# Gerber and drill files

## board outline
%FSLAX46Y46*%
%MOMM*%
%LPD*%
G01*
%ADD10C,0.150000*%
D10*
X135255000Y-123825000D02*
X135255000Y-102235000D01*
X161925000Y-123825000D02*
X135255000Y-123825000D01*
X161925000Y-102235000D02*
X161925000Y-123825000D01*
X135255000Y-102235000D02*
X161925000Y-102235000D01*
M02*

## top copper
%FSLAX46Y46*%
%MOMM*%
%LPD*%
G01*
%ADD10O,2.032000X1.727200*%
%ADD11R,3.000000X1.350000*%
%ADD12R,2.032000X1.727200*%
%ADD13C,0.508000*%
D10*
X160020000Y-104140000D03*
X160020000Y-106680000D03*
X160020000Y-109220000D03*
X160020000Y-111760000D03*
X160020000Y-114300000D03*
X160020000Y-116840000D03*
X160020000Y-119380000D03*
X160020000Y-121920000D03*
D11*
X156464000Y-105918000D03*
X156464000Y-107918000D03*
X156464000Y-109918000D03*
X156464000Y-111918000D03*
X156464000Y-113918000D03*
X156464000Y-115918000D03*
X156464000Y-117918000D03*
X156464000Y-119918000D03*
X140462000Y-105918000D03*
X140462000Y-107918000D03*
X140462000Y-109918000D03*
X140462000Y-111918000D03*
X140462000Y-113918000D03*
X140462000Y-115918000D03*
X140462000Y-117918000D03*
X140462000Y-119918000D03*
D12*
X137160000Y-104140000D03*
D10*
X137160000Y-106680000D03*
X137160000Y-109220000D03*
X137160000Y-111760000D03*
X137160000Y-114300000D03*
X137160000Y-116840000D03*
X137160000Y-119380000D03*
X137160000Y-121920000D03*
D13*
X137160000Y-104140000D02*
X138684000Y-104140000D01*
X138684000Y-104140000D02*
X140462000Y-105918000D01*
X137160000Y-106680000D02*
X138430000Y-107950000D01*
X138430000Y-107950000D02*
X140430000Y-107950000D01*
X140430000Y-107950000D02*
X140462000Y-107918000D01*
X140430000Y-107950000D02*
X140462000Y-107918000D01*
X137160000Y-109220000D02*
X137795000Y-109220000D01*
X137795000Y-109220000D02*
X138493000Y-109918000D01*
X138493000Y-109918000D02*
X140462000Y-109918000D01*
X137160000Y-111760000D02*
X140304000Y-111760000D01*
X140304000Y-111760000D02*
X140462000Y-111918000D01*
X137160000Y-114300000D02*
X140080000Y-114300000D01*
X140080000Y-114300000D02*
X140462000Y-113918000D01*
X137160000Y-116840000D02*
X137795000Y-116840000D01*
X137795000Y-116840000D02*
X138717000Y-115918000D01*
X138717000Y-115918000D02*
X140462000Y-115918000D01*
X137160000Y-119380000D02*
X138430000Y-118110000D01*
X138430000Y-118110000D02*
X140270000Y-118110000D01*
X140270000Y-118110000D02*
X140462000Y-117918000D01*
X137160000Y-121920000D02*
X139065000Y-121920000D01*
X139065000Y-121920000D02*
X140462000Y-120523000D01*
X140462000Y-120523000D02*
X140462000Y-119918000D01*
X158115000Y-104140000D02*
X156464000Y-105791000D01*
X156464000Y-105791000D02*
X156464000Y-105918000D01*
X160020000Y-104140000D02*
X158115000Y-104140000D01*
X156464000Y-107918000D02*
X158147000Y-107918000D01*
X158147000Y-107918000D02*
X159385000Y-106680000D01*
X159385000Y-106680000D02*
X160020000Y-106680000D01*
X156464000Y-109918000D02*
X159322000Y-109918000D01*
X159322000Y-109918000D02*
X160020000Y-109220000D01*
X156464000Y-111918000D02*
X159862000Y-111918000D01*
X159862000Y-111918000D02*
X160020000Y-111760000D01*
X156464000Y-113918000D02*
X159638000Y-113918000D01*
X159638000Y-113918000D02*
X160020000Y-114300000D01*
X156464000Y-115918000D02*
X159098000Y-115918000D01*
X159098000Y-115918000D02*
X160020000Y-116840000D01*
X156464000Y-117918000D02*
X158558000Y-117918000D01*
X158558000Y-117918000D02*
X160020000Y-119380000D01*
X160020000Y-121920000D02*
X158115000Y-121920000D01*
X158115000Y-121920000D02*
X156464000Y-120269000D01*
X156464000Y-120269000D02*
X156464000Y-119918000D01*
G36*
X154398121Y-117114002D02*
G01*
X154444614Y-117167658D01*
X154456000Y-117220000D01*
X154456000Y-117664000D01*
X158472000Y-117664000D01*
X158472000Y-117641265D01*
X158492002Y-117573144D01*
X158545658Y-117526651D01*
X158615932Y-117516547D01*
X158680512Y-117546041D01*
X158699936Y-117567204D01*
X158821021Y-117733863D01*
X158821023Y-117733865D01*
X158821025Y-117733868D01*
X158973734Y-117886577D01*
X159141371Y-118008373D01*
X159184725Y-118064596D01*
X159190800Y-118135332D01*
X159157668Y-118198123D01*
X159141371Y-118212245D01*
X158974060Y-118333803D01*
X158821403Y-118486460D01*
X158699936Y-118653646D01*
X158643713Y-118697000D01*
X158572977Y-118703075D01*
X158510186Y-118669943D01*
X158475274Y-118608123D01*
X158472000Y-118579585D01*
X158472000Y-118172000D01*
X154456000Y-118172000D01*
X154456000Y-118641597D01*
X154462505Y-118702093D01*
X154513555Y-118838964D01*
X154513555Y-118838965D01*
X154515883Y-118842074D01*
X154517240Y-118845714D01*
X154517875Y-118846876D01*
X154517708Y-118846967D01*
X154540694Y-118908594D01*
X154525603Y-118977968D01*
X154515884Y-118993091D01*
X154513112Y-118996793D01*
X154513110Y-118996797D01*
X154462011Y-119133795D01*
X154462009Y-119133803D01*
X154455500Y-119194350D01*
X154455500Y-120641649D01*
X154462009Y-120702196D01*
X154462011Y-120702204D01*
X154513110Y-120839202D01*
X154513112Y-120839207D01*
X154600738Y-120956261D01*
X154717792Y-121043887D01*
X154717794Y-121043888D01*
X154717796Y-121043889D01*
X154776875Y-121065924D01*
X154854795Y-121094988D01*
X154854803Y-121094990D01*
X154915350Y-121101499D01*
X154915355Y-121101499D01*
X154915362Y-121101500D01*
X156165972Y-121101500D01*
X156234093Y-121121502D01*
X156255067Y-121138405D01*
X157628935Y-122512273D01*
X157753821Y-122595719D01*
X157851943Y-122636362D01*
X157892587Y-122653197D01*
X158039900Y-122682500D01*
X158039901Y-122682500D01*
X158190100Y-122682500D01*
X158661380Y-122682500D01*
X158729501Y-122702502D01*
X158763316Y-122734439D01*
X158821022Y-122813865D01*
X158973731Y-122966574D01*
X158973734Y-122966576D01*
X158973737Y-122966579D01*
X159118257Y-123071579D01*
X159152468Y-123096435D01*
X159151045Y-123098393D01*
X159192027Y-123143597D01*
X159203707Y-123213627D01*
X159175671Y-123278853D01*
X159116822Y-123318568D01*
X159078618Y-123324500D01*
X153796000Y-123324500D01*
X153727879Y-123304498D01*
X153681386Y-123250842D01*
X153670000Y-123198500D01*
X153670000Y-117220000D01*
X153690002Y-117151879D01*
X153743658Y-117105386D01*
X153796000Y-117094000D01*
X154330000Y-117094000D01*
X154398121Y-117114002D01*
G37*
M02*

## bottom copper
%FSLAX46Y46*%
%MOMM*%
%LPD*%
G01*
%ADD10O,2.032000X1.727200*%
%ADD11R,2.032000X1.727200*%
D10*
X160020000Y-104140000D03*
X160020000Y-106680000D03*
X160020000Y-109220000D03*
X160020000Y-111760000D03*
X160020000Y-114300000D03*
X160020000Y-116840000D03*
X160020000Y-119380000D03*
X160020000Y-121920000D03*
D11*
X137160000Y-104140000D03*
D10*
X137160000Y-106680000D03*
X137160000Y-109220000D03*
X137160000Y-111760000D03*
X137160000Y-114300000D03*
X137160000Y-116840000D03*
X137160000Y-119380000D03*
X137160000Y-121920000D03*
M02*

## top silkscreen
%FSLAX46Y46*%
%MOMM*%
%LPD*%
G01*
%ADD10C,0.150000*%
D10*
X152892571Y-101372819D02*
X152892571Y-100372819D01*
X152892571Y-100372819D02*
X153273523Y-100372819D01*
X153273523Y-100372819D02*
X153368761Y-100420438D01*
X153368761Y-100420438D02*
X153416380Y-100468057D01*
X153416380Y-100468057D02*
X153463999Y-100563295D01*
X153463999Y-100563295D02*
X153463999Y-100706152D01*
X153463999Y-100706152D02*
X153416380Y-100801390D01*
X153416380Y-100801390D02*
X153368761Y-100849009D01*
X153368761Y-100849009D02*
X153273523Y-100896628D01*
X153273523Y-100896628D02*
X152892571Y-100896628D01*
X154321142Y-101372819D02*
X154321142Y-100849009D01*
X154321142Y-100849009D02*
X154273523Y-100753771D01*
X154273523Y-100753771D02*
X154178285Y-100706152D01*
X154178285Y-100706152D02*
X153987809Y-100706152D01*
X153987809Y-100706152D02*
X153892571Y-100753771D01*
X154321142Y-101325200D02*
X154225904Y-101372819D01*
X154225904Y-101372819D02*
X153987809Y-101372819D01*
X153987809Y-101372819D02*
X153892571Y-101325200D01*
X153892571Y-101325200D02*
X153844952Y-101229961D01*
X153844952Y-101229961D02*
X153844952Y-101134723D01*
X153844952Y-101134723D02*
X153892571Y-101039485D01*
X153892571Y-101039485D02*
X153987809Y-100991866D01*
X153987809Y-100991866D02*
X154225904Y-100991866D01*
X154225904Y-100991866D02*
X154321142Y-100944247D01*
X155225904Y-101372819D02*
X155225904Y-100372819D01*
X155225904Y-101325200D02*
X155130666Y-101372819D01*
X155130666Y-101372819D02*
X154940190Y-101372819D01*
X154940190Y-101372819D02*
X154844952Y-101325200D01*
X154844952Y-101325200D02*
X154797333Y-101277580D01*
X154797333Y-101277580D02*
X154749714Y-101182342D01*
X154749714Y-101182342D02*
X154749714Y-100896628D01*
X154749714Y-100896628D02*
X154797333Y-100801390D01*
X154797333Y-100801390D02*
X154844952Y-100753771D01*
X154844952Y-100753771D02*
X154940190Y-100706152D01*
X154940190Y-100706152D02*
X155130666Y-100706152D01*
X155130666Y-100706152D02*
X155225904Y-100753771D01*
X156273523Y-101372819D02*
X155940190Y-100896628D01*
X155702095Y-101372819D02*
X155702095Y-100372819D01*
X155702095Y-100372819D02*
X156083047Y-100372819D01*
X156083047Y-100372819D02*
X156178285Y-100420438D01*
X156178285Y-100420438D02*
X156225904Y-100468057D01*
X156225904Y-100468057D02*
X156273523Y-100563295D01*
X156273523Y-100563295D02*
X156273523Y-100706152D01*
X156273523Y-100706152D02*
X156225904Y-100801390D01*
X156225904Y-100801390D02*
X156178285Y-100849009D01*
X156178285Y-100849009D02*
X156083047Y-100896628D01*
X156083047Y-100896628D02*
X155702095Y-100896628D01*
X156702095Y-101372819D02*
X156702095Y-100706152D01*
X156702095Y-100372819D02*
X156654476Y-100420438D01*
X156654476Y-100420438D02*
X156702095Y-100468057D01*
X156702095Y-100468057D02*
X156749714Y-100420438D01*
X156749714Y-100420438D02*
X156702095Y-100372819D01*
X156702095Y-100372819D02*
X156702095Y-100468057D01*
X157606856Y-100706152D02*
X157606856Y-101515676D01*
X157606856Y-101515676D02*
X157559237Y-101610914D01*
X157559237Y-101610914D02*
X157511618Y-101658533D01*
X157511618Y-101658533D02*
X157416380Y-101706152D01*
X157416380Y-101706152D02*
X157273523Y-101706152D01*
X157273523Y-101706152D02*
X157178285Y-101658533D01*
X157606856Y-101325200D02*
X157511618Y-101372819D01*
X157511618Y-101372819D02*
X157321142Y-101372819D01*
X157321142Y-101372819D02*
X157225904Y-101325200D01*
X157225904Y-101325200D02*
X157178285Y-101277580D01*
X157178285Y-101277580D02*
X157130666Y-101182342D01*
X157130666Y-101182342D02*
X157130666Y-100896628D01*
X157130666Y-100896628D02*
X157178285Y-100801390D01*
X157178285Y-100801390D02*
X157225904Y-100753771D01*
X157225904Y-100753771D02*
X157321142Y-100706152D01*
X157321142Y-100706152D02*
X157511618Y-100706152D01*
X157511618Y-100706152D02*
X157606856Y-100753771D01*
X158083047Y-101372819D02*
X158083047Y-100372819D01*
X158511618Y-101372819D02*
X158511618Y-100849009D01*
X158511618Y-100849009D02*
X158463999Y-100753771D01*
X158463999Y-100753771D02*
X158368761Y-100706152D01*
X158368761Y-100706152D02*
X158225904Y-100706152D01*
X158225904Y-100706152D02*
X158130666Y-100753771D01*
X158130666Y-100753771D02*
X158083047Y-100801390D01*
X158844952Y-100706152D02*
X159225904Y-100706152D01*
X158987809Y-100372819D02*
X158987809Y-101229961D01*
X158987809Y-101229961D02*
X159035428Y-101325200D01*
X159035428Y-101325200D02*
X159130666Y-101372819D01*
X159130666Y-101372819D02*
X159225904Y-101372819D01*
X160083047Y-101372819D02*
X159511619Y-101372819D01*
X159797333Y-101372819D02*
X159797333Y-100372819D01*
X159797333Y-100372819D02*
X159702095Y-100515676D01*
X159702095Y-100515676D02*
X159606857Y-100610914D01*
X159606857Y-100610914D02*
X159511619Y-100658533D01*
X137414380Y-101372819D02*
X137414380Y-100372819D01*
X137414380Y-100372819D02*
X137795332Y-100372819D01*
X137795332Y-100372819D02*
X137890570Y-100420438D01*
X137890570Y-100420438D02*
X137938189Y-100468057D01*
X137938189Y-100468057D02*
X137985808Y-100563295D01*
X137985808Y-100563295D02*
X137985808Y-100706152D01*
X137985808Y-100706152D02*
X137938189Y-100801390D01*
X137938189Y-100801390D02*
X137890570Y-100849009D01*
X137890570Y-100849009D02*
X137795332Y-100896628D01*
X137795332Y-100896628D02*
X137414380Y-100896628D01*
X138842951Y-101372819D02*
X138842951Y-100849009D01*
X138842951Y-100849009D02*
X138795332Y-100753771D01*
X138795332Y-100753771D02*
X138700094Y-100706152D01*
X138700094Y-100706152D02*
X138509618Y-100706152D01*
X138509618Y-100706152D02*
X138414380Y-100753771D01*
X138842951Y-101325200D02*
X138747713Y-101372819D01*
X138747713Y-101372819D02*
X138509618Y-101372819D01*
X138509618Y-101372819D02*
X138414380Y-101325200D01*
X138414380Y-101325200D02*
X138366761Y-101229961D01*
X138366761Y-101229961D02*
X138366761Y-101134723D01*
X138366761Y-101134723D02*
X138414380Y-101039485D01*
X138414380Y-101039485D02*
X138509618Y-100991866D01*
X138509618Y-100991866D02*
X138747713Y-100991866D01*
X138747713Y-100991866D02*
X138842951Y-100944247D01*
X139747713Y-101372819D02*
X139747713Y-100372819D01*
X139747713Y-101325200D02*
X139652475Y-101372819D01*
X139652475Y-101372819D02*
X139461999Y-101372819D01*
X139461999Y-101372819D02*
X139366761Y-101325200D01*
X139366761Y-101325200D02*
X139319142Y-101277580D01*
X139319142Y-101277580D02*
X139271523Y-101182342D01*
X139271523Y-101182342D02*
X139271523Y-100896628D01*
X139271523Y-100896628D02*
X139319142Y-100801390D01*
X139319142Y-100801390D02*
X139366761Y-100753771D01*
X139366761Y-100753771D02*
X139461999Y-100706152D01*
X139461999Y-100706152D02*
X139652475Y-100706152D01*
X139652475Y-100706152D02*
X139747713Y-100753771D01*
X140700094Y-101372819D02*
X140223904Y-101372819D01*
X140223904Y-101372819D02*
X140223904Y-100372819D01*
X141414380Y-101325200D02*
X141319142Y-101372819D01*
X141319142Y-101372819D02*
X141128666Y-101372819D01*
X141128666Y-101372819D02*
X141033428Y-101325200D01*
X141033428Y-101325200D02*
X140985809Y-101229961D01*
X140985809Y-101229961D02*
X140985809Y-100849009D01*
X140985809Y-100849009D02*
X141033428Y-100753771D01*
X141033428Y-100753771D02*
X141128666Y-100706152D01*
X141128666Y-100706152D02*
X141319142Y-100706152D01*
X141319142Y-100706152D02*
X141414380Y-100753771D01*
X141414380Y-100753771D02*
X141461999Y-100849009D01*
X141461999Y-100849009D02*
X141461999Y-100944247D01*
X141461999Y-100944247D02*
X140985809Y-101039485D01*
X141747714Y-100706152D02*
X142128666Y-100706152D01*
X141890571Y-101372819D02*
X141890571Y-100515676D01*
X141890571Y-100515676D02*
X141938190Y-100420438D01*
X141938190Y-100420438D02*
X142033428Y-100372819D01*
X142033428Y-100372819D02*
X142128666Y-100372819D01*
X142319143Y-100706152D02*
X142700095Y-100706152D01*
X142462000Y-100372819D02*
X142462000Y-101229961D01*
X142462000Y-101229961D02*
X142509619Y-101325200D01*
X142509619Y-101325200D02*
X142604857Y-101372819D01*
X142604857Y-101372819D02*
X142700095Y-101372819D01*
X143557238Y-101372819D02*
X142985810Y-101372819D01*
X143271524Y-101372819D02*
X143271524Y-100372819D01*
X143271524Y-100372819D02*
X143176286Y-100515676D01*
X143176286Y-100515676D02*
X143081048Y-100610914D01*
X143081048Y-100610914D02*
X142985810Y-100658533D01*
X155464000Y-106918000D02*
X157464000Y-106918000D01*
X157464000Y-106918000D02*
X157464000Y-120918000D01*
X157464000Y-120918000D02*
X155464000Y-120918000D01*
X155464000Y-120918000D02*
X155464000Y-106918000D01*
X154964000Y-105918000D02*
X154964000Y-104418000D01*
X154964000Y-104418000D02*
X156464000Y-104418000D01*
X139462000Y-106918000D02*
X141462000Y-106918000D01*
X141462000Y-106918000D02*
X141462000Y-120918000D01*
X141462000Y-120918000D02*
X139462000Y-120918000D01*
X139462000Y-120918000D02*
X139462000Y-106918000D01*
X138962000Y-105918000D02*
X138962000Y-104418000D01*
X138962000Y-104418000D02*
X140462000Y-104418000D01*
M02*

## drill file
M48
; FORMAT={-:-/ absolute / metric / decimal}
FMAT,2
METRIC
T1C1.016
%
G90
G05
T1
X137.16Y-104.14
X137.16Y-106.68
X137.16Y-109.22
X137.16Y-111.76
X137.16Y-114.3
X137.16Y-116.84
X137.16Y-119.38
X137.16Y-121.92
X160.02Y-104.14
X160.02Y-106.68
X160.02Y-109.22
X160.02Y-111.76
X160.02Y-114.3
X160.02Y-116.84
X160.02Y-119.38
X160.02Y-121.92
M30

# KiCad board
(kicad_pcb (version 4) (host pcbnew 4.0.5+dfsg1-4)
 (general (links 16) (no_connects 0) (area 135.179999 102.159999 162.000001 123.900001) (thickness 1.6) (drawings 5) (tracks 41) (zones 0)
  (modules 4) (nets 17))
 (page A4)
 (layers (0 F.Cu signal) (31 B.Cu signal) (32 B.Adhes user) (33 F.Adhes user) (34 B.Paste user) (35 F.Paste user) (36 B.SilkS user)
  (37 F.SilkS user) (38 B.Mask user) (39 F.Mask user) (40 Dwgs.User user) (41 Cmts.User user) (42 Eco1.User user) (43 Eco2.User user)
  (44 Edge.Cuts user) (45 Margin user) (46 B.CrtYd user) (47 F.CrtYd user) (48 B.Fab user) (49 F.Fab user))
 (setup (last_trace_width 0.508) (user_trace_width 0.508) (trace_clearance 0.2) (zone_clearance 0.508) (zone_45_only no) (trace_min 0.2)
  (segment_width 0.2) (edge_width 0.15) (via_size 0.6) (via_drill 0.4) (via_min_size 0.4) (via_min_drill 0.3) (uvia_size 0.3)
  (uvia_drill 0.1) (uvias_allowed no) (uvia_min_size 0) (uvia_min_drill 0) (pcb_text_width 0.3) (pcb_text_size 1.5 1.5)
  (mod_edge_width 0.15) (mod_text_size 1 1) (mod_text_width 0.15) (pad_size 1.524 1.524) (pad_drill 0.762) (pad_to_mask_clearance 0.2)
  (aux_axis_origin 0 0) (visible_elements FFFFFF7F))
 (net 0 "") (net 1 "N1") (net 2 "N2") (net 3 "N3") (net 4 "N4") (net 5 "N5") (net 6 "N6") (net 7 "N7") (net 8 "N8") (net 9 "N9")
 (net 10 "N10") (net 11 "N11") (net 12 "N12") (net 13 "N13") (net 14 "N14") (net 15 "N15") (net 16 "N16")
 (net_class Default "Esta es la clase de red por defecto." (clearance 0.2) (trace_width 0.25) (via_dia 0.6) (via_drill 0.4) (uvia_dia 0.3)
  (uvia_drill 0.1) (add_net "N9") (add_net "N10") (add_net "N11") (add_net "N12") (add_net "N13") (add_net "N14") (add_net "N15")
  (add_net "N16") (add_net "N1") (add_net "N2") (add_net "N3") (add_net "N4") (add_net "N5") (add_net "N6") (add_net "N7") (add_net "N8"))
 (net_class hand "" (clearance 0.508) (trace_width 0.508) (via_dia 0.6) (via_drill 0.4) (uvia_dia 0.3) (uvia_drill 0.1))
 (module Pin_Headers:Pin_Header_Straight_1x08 (layer B.Cu) (at 160.02 104.14 180)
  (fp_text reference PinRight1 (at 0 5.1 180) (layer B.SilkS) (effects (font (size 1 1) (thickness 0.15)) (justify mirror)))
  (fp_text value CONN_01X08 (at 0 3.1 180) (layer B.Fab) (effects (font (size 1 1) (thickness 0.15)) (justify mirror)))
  (pad 1 thru_hole oval (at 0 0 180) (size 2.032 1.7272) (drill 1.016) (layers *.Cu *.Mask) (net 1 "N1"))
  (pad 2 thru_hole oval (at 0 -2.54 180) (size 2.032 1.7272) (drill 1.016) (layers *.Cu *.Mask) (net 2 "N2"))
  (pad 3 thru_hole oval (at 0 -5.08 180) (size 2.032 1.7272) (drill 1.016) (layers *.Cu *.Mask) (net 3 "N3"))
  (pad 4 thru_hole oval (at 0 -7.62 180) (size 2.032 1.7272) (drill 1.016) (layers *.Cu *.Mask) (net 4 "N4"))
  (pad 5 thru_hole oval (at 0 -10.16 180) (size 2.032 1.7272) (drill 1.016) (layers *.Cu *.Mask) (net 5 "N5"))
  (pad 6 thru_hole oval (at 0 -12.7 180) (size 2.032 1.7272) (drill 1.016) (layers *.Cu *.Mask) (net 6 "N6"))
  (pad 7 thru_hole oval (at 0 -15.24 180) (size 2.032 1.7272) (drill 1.016) (layers *.Cu *.Mask) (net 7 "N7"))
  (pad 8 thru_hole oval (at 0 -17.78 180) (size 2.032 1.7272) (drill 1.016) (layers *.Cu *.Mask) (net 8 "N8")))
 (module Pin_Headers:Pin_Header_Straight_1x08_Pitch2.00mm (layer F.Cu) (at 156.464 105.918)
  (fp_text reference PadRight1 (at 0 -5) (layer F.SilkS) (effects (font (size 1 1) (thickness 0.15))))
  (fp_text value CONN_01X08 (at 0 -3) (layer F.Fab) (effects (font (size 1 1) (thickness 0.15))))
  (fp_line (start -1 1) (end 1 1) (layer F.SilkS) (width 0.15))
  (fp_line (start 1 1) (end 1 15) (layer F.SilkS) (width 0.15))
  (fp_line (start 1 15) (end -1 15) (layer F.SilkS) (width 0.15))
  (fp_line (start -1 15) (end -1 1) (layer F.SilkS) (width 0.15))
  (fp_line (start -1.5 0) (end -1.5 -1.5) (layer F.SilkS) (width 0.15))
  (fp_line (start -1.5 -1.5) (end 0 -1.5) (layer F.SilkS) (width 0.15))
  (pad 1 smd rect (at 0 0) (size 3 1.35) (layers F.Cu F.Paste F.Mask) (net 1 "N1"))
  (pad 2 smd rect (at 0 2) (size 3 1.35) (layers F.Cu F.Paste F.Mask) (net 2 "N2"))
  (pad 3 smd rect (at 0 4) (size 3 1.35) (layers F.Cu F.Paste F.Mask) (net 3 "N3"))
  (pad 4 smd rect (at 0 6) (size 3 1.35) (layers F.Cu F.Paste F.Mask) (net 4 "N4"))
  (pad 5 smd rect (at 0 8) (size 3 1.35) (layers F.Cu F.Paste F.Mask) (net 5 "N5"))
  (pad 6 smd rect (at 0 10) (size 3 1.35) (layers F.Cu F.Paste F.Mask) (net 6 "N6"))
  (pad 7 smd rect (at 0 12) (size 3 1.35) (layers F.Cu F.Paste F.Mask) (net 7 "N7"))
  (pad 8 smd rect (at 0 14) (size 3 1.35) (layers F.Cu F.Paste F.Mask) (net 8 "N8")))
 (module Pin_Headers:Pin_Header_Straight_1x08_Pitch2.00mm (layer F.Cu) (at 140.462 105.918)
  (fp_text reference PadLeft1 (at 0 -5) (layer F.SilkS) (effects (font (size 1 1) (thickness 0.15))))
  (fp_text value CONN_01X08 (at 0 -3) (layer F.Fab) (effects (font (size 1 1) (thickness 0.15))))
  (fp_line (start -1 1) (end 1 1) (layer F.SilkS) (width 0.15))
  (fp_line (start 1 1) (end 1 15) (layer F.SilkS) (width 0.15))
  (fp_line (start 1 15) (end -1 15) (layer F.SilkS) (width 0.15))
  (fp_line (start -1 15) (end -1 1) (layer F.SilkS) (width 0.15))
  (fp_line (start -1.5 0) (end -1.5 -1.5) (layer F.SilkS) (width 0.15))
  (fp_line (start -1.5 -1.5) (end 0 -1.5) (layer F.SilkS) (width 0.15))
  (pad 1 smd rect (at 0 0) (size 3 1.35) (layers F.Cu F.Paste F.Mask) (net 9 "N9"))
  (pad 2 smd rect (at 0 2) (size 3 1.35) (layers F.Cu F.Paste F.Mask) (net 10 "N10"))
  (pad 3 smd rect (at 0 4) (size 3 1.35) (layers F.Cu F.Paste F.Mask) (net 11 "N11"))
  (pad 4 smd rect (at 0 6) (size 3 1.35) (layers F.Cu F.Paste F.Mask) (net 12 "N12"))
  (pad 5 smd rect (at 0 8) (size 3 1.35) (layers F.Cu F.Paste F.Mask) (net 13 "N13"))
  (pad 6 smd rect (at 0 10) (size 3 1.35) (layers F.Cu F.Paste F.Mask) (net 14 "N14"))
  (pad 7 smd rect (at 0 12) (size 3 1.35) (layers F.Cu F.Paste F.Mask) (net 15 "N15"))
  (pad 8 smd rect (at 0 14) (size 3 1.35) (layers F.Cu F.Paste F.Mask) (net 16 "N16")))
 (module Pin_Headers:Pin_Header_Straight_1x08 (layer B.Cu) (at 137.16 104.14 180)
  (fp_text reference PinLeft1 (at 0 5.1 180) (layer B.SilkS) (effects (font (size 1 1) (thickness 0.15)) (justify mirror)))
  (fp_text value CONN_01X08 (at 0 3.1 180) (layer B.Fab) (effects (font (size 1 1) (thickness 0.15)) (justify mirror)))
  (pad 1 thru_hole rect (at 0 0 180) (size 2.032 1.7272) (drill 1.016) (layers *.Cu *.Mask) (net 9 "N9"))
  (pad 2 thru_hole oval (at 0 -2.54 180) (size 2.032 1.7272) (drill 1.016) (layers *.Cu *.Mask) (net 10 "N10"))
  (pad 3 thru_hole oval (at 0 -5.08 180) (size 2.032 1.7272) (drill 1.016) (layers *.Cu *.Mask) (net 11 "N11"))
  (pad 4 thru_hole oval (at 0 -7.62 180) (size 2.032 1.7272) (drill 1.016) (layers *.Cu *.Mask) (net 12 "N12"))
  (pad 5 thru_hole oval (at 0 -10.16 180) (size 2.032 1.7272) (drill 1.016) (layers *.Cu *.Mask) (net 13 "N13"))
  (pad 6 thru_hole oval (at 0 -12.7 180) (size 2.032 1.7272) (drill 1.016) (layers *.Cu *.Mask) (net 14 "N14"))
  (pad 7 thru_hole oval (at 0 -15.24 180) (size 2.032 1.7272) (drill 1.016) (layers *.Cu *.Mask) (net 15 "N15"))
  (pad 8 thru_hole oval (at 0 -17.78 180) (size 2.032 1.7272) (drill 1.016) (layers *.Cu *.Mask) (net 16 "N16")))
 (gr_line (start 135.255 123.825) (end 135.255 102.235) (angle 90) (layer Edge.Cuts) (width 0.15))
 (gr_line (start 161.925 123.825) (end 135.255 123.825) (angle 90) (layer Edge.Cuts) (width 0.15))
 (gr_line (start 161.925 102.235) (end 161.925 123.825) (angle 90) (layer Edge.Cuts) (width 0.15))
 (gr_line (start 135.255 102.235) (end 161.925 102.235) (angle 90) (layer Edge.Cuts) (width 0.15))
 (segment (start 137.16 104.14) (end 138.684 104.14) (width 0.508) (layer F.Cu) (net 9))
 (segment (start 138.684 104.14) (end 140.462 105.918) (width 0.508) (layer F.Cu) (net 9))
 (segment (start 137.16 106.68) (end 138.43 107.95) (width 0.508) (layer F.Cu) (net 10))
 (segment (start 138.43 107.95) (end 140.43 107.95) (width 0.508) (layer F.Cu) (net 10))
 (segment (start 140.43 107.95) (end 140.462 107.918) (width 0.508) (layer F.Cu) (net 10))
 (segment (start 140.43 107.95) (end 140.462 107.918) (width 0.508) (layer F.Cu) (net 10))
 (segment (start 137.16 109.22) (end 137.795 109.22) (width 0.508) (layer F.Cu) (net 11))
 (segment (start 137.795 109.22) (end 138.493 109.918) (width 0.508) (layer F.Cu) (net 11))
 (segment (start 138.493 109.918) (end 140.462 109.918) (width 0.508) (layer F.Cu) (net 11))
 (segment (start 137.16 111.76) (end 140.304 111.76) (width 0.508) (layer F.Cu) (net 12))
 (segment (start 140.304 111.76) (end 140.462 111.918) (width 0.508) (layer F.Cu) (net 12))
 (segment (start 137.16 114.3) (end 140.08 114.3) (width 0.508) (layer F.Cu) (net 13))
 (segment (start 140.08 114.3) (end 140.462 113.918) (width 0.508) (layer F.Cu) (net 13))
 (segment (start 137.16 116.84) (end 137.795 116.84) (width 0.508) (layer F.Cu) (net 14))
 (segment (start 137.795 116.84) (end 138.717 115.918) (width 0.508) (layer F.Cu) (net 14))
 (segment (start 138.717 115.918) (end 140.462 115.918) (width 0.508) (layer F.Cu) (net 14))
 (segment (start 137.16 119.38) (end 138.43 118.11) (width 0.508) (layer F.Cu) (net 15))
 (segment (start 138.43 118.11) (end 140.27 118.11) (width 0.508) (layer F.Cu) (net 15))
 (segment (start 140.27 118.11) (end 140.462 117.918) (width 0.508) (layer F.Cu) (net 15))
 (segment (start 137.16 121.92) (end 139.065 121.92) (width 0.508) (layer F.Cu) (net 16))
 (segment (start 139.065 121.92) (end 140.462 120.523) (width 0.508) (layer F.Cu) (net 16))
 (segment (start 140.462 120.523) (end 140.462 119.918) (width 0.508) (layer F.Cu) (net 16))
 (segment (start 158.115 104.14) (end 156.464 105.791) (width 0.508) (layer F.Cu) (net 1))
 (segment (start 156.464 105.791) (end 156.464 105.918) (width 0.508) (layer F.Cu) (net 1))
 (segment (start 160.02 104.14) (end 158.115 104.14) (width 0.508) (layer F.Cu) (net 1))
 (segment (start 156.464 107.918) (end 158.147 107.918) (width 0.508) (layer F.Cu) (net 2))
 (segment (start 158.147 107.918) (end 159.385 106.68) (width 0.508) (layer F.Cu) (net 2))
 (segment (start 159.385 106.68) (end 160.02 106.68) (width 0.508) (layer F.Cu) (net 2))
 (segment (start 156.464 109.918) (end 159.322 109.918) (width 0.508) (layer F.Cu) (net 3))
 (segment (start 159.322 109.918) (end 160.02 109.22) (width 0.508) (layer F.Cu) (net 3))
 (segment (start 156.464 111.918) (end 159.862 111.918) (width 0.508) (layer F.Cu) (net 4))
 (segment (start 159.862 111.918) (end 160.02 111.76) (width 0.508) (layer F.Cu) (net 4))
 (segment (start 156.464 113.918) (end 159.638 113.918) (width 0.508) (layer F.Cu) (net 5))
 (segment (start 159.638 113.918) (end 160.02 114.3) (width 0.508) (layer F.Cu) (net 5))
 (segment (start 156.464 115.918) (end 159.098 115.918) (width 0.508) (layer F.Cu) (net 6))
 (segment (start 159.098 115.918) (end 160.02 116.84) (width 0.508) (layer F.Cu) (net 6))
 (segment (start 156.464 117.918) (end 158.558 117.918) (width 0.508) (layer F.Cu) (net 7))
 (segment (start 158.558 117.918) (end 160.02 119.38) (width 0.508) (layer F.Cu) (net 7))
 (segment (start 160.02 121.92) (end 158.115 121.92) (width 0.508) (layer F.Cu) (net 8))
 (segment (start 158.115 121.92) (end 156.464 120.269) (width 0.508) (layer F.Cu) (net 8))
 (segment (start 156.464 120.269) (end 156.464 119.918) (width 0.508) (layer F.Cu) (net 8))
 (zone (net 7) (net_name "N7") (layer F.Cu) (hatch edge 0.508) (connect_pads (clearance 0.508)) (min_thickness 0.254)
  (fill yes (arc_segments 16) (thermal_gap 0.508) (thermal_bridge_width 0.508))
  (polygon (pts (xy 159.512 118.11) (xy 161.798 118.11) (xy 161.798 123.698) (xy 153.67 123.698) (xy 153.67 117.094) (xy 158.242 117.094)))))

